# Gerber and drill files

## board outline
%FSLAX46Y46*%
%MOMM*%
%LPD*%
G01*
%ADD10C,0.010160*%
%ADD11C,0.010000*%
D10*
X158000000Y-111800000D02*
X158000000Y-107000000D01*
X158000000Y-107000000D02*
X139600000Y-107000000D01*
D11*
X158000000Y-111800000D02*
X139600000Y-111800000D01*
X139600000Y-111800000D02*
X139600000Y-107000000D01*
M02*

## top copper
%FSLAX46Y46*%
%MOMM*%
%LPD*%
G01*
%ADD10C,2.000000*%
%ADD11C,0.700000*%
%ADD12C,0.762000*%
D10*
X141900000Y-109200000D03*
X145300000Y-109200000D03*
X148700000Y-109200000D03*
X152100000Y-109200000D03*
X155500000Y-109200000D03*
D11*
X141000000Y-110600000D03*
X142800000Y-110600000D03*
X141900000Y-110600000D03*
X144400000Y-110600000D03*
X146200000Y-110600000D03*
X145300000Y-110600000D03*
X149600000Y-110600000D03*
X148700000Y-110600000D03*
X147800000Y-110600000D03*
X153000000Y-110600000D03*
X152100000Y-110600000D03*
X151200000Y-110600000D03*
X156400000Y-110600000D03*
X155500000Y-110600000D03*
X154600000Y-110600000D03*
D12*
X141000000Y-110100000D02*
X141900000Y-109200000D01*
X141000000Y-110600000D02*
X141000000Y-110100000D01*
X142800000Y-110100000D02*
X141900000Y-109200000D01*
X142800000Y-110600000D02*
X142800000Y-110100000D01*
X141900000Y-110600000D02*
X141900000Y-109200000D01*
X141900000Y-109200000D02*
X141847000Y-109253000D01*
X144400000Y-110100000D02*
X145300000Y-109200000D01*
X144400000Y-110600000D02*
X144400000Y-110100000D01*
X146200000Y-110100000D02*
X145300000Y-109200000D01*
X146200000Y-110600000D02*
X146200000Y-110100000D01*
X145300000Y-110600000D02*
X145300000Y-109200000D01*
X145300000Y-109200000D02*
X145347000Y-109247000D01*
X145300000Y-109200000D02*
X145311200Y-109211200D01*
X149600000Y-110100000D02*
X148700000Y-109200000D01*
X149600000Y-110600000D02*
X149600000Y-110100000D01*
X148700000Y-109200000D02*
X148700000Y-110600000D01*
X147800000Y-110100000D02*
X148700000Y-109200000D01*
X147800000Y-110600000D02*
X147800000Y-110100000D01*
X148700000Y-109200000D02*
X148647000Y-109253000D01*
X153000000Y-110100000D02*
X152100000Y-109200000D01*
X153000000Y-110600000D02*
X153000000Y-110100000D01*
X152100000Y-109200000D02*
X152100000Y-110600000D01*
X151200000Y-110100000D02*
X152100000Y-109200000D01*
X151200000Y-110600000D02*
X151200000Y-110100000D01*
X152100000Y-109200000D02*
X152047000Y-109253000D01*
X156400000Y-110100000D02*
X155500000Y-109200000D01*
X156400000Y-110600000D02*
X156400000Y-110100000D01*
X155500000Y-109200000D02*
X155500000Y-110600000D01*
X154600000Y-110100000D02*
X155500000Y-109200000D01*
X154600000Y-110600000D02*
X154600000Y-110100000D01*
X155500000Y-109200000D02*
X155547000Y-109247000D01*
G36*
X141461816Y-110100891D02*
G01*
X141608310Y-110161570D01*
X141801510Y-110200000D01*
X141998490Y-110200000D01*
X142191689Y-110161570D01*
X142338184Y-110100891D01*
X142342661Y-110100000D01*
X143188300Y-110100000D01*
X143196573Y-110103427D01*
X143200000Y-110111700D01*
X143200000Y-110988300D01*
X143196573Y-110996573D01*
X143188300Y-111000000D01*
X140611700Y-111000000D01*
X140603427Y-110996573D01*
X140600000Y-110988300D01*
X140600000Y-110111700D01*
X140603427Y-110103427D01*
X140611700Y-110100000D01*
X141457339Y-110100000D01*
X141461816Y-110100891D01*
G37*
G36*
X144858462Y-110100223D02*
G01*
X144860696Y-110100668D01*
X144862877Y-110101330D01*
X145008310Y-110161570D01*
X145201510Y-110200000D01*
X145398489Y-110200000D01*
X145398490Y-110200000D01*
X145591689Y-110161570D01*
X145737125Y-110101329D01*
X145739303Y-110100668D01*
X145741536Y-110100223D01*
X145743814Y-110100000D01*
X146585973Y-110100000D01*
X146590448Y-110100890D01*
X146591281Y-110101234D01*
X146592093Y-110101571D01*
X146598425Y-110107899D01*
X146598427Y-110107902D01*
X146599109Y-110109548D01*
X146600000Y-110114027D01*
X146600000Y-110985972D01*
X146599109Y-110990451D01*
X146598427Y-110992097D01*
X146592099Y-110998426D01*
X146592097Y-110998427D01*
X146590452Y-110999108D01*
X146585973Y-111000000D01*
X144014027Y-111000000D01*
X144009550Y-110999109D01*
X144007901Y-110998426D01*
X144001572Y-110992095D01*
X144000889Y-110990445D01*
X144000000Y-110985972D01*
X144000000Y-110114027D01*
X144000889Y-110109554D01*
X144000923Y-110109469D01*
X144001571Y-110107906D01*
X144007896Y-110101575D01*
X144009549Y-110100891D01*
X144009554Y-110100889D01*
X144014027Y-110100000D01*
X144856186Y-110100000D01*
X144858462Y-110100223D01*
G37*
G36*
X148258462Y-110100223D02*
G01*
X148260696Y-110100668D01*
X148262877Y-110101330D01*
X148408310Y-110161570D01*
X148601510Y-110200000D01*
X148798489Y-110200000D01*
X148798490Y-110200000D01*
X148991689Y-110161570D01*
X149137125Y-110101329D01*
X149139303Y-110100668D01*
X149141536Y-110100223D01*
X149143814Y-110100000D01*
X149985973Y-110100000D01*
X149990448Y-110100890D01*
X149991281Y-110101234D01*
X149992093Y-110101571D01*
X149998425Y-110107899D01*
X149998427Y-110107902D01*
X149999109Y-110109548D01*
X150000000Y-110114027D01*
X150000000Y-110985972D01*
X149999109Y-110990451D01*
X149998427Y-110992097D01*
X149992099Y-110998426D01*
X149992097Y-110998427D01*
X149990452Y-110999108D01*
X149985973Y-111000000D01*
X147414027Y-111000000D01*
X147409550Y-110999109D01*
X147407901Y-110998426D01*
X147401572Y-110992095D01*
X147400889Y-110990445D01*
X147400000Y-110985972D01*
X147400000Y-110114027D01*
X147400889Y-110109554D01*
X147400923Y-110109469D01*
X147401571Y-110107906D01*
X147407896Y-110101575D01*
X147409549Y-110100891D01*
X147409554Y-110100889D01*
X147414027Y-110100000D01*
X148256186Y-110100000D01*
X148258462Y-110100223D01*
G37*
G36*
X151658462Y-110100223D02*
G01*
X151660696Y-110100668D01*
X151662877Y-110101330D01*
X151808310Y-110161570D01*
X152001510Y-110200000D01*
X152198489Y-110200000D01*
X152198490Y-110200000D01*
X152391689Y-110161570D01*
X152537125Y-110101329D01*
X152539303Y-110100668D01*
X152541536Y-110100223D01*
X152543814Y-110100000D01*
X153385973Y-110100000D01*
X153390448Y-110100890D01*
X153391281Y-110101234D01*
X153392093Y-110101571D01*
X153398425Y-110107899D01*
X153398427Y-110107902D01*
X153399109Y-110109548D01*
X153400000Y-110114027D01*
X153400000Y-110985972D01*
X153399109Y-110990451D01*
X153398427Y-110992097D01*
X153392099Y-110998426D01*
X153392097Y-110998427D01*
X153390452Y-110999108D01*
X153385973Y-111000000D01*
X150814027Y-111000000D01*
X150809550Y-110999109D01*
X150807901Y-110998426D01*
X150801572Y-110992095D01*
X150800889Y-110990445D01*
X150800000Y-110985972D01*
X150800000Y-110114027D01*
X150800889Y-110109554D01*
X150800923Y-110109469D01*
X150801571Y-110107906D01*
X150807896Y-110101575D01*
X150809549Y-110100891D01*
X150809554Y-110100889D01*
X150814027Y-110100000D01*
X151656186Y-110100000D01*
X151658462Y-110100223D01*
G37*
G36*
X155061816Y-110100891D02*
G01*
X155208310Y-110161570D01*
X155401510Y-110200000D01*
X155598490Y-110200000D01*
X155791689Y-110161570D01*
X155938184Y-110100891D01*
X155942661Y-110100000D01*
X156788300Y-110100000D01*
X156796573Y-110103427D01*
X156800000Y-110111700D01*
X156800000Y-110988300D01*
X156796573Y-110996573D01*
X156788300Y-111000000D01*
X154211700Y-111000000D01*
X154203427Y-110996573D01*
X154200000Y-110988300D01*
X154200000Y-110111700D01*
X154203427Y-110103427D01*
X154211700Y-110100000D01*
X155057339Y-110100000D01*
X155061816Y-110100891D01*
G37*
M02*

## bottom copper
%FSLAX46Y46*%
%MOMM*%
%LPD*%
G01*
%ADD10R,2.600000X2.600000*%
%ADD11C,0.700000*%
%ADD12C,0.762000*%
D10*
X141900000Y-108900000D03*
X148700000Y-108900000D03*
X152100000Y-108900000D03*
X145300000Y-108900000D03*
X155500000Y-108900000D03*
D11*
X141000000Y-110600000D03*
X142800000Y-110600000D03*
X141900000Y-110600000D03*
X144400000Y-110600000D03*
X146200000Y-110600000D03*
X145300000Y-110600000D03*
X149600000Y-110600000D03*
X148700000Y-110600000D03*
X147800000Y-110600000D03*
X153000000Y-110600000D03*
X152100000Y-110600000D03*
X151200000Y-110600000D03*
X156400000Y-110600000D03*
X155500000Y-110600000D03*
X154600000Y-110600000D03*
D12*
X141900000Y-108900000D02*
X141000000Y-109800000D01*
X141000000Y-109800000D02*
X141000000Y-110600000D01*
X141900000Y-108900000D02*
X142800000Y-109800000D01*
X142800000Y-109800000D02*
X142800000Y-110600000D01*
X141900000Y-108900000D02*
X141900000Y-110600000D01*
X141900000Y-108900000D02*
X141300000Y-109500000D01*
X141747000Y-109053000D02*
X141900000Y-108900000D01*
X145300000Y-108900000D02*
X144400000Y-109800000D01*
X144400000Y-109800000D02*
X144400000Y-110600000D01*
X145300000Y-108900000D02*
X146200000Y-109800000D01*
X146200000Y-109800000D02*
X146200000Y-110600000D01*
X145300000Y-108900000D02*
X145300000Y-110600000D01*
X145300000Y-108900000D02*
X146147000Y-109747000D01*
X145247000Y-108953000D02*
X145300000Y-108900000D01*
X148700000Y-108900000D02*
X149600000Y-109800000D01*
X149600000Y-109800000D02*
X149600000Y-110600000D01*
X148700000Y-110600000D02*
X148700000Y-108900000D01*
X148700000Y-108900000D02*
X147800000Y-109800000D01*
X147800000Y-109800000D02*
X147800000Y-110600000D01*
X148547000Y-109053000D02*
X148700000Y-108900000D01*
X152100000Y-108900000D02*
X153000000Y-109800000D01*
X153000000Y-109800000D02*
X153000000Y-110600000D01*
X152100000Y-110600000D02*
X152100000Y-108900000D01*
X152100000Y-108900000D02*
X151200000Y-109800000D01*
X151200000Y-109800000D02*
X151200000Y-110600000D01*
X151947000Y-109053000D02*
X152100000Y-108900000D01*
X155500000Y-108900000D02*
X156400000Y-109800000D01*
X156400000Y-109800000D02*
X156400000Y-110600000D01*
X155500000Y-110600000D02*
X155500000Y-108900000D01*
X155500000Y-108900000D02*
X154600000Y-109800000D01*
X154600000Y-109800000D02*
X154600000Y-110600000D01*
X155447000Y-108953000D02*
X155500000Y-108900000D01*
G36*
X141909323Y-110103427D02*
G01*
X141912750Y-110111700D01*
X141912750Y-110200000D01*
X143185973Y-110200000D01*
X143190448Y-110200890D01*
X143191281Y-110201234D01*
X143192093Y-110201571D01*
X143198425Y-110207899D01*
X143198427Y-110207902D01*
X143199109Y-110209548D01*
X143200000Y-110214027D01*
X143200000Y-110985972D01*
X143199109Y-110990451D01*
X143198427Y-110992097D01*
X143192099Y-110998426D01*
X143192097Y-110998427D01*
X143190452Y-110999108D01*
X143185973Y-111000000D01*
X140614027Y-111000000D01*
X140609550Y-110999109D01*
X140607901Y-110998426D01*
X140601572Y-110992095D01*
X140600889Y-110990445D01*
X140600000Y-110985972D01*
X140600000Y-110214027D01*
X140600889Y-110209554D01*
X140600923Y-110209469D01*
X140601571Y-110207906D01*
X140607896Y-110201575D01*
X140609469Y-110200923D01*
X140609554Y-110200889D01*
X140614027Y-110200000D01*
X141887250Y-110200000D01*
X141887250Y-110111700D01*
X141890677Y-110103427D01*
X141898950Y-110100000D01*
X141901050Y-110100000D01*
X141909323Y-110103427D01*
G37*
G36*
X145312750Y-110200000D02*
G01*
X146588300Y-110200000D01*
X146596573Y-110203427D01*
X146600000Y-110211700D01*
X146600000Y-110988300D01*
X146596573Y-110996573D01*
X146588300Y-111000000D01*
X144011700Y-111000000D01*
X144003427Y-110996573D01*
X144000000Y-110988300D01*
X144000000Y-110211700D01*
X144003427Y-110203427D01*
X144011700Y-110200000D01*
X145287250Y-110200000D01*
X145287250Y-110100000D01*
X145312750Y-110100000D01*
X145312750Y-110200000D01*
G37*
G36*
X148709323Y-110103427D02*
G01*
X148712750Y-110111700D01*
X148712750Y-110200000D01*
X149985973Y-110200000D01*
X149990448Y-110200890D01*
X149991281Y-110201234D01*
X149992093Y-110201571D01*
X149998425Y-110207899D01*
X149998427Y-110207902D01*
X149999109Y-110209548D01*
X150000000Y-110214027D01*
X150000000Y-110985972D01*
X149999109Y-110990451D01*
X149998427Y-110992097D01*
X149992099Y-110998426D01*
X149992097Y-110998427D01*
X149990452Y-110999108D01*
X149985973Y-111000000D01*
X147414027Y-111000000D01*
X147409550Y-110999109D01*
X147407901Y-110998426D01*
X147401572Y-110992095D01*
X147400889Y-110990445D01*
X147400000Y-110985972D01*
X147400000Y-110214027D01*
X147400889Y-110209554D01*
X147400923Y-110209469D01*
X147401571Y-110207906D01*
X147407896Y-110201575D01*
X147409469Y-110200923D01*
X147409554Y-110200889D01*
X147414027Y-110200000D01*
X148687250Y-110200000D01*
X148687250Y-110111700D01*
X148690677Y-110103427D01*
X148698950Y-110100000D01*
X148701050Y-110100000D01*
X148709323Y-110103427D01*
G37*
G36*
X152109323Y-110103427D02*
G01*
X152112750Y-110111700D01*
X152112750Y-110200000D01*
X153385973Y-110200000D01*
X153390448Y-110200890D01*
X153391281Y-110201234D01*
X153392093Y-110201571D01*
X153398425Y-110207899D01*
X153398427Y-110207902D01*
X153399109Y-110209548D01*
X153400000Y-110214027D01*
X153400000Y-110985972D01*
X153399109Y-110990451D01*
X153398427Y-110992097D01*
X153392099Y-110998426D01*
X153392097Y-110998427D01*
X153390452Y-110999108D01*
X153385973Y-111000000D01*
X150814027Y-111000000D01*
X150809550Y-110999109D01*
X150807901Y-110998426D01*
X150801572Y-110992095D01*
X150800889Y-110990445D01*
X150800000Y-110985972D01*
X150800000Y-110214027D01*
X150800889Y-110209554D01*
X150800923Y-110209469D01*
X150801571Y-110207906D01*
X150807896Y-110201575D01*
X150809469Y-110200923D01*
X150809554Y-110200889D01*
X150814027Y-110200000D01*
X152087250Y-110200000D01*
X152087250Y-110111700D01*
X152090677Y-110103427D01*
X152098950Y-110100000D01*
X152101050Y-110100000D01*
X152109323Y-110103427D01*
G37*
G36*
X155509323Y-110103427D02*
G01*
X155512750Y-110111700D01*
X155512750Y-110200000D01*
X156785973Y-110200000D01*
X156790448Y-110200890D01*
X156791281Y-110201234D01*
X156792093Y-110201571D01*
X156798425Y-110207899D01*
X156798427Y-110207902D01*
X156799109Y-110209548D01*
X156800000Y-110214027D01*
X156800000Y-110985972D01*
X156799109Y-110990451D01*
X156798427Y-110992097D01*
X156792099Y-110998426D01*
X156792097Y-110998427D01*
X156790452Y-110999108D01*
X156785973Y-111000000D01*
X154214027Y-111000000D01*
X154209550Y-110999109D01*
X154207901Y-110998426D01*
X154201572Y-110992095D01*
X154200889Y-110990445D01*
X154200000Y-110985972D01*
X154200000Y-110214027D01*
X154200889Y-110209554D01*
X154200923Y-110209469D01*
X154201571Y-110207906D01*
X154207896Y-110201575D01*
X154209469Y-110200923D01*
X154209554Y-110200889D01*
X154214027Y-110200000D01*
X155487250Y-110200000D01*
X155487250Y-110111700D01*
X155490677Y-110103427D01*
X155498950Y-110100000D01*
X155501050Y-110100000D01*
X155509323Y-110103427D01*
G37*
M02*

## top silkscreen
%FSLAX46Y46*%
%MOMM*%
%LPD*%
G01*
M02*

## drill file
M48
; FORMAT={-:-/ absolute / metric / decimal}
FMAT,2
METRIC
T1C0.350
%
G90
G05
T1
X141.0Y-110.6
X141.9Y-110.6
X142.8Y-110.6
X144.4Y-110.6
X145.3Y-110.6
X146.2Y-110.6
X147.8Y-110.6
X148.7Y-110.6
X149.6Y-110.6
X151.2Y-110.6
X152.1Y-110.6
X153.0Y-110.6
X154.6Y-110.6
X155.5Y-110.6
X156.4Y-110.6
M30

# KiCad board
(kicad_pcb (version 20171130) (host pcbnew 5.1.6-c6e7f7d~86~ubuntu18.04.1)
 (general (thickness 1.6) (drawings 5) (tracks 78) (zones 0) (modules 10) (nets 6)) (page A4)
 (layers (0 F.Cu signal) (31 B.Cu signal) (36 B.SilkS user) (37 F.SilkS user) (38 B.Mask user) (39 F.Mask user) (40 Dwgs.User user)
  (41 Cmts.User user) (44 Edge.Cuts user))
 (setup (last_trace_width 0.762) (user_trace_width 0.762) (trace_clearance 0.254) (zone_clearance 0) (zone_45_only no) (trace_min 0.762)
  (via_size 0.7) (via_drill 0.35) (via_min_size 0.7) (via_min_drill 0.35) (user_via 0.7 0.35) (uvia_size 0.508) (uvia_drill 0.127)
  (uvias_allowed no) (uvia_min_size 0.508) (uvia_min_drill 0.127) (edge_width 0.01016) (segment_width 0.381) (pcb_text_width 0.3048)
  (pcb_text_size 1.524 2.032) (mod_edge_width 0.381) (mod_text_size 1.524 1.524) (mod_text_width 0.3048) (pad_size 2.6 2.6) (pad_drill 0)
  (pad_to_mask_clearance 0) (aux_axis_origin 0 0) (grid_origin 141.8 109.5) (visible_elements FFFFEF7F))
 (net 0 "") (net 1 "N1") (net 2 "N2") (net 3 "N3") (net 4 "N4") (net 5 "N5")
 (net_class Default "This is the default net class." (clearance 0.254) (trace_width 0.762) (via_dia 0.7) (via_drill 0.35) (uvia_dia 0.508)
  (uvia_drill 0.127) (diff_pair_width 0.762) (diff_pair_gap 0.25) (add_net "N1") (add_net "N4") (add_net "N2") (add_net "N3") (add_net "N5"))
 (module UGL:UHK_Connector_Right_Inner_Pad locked (layer B.Cu) (at 146.31 108.9)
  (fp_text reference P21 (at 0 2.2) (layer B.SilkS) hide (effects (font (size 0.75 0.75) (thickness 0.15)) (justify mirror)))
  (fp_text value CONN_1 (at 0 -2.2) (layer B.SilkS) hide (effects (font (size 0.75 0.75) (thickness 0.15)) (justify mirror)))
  (pad 1 smd rect (at -4.41 0) (size 2.6 2.6) (layers B.Cu B.Mask) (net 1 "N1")))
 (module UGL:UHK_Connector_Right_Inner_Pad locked (layer B.Cu) (at 151.15 108.9)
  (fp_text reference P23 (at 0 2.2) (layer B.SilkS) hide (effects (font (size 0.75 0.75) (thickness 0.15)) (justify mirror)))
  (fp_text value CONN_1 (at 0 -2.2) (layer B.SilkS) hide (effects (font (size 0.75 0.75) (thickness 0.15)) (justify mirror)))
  (pad 1 smd rect (at -2.45 0) (size 2.6 2.6) (layers B.Cu B.Mask) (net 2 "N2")))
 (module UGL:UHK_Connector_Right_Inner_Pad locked (layer B.Cu) (at 153.57 108.9)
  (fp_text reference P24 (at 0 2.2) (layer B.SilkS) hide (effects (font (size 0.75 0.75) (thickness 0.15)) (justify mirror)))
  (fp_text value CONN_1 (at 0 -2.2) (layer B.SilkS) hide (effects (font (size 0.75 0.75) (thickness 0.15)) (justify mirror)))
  (pad 1 smd rect (at -1.47 0) (size 2.6 2.6) (layers B.Cu B.Mask) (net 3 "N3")))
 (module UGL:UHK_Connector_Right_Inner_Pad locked (layer B.Cu) (at 148.73 108.9)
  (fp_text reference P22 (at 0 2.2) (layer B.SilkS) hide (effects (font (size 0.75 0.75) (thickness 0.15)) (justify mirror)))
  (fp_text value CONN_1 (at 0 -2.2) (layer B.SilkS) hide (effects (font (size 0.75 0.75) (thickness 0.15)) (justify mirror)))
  (pad 1 smd rect (at -3.43 0) (size 2.6 2.6) (layers B.Cu B.Mask) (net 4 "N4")))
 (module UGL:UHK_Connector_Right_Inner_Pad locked (layer B.Cu) (at 155.99 108.9)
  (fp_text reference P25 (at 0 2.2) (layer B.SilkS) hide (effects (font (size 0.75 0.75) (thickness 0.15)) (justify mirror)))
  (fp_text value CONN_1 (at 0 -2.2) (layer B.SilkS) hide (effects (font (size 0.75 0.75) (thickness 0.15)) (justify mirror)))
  (pad 1 smd rect (at -0.49 0) (size 2.6 2.6) (layers B.Cu B.Mask) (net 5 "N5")))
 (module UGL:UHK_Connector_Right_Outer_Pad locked (layer F.Cu) (at 141.9 109.2)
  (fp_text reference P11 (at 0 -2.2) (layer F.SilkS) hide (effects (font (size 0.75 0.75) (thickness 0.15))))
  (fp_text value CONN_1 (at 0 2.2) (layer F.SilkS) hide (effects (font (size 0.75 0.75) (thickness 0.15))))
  (pad 1 smd circle (at 0 0) (size 2 2) (layers F.Cu F.Mask) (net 1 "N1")))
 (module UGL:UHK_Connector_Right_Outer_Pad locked (layer F.Cu) (at 145.3 109.2)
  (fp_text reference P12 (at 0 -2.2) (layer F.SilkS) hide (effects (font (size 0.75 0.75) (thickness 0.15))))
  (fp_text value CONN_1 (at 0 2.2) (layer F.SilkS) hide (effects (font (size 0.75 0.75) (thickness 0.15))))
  (pad 1 smd circle (at 0 0) (size 2 2) (layers F.Cu F.Mask) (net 4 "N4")))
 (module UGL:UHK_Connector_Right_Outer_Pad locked (layer F.Cu) (at 148.7 109.2)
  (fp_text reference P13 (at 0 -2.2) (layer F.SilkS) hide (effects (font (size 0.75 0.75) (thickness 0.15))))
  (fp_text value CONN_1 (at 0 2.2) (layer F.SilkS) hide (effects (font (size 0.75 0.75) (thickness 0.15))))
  (pad 1 smd circle (at 0 0) (size 2 2) (layers F.Cu F.Mask) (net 2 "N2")))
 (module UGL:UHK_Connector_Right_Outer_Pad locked (layer F.Cu) (at 152.1 109.2)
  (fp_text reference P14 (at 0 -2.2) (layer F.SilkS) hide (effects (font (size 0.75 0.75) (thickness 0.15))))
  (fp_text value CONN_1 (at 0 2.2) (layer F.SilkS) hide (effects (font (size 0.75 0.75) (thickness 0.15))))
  (pad 1 smd circle (at 0 0) (size 2 2) (layers F.Cu F.Mask) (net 3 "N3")))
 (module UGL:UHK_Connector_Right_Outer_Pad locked (layer F.Cu) (at 155.5 109.2)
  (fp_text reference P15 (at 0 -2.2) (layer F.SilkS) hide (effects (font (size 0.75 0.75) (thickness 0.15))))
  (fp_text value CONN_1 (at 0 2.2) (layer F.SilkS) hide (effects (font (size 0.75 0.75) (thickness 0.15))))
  (pad 1 smd circle (at 0 0) (size 2 2) (layers F.Cu F.Mask) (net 5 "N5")))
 (gr_line (start 158 111.8) (end 158 107) (layer Edge.Cuts) (width 0.01016))
 (gr_line (start 158 107) (end 139.6 107) (layer Edge.Cuts) (width 0.01016))
 (gr_line (start 158 111.8) (end 139.6 111.8) (angle 90) (layer Edge.Cuts) (width 0.01))
 (gr_line (start 139.6 111.8) (end 139.6 107) (angle 90) (layer Edge.Cuts) (width 0.01))
 (segment (start 141.9 108.9) (end 141 109.8) (width 0.762) (layer B.Cu) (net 1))
 (segment (start 141 109.8) (end 141 110.6) (width 0.762) (layer B.Cu) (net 1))
 (segment (start 141 110.1) (end 141.9 109.2) (width 0.762) (layer F.Cu) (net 1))
 (segment (start 141 110.6) (end 141 110.1) (width 0.762) (layer F.Cu) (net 1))
 (via (at 141 110.6) (size 0.7) (drill 0.35) (layers F.Cu B.Cu) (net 1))
 (segment (start 141.9 108.9) (end 142.8 109.8) (width 0.762) (layer B.Cu) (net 1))
 (segment (start 142.8 109.8) (end 142.8 110.6) (width 0.762) (layer B.Cu) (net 1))
 (segment (start 142.8 110.1) (end 141.9 109.2) (width 0.762) (layer F.Cu) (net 1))
 (segment (start 142.8 110.6) (end 142.8 110.1) (width 0.762) (layer F.Cu) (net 1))
 (via (at 142.8 110.6) (size 0.7) (drill 0.35) (layers F.Cu B.Cu) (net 1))
 (segment (start 141.9 108.9) (end 141.9 110.6) (width 0.762) (layer B.Cu) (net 1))
 (segment (start 141.9 110.6) (end 141.9 109.2) (width 0.762) (layer F.Cu) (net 1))
 (via (at 141.9 110.6) (size 0.7) (drill 0.35) (layers F.Cu B.Cu) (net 1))
 (segment (start 141.9 108.9) (end 141.3 109.5) (width 0.762) (layer B.Cu) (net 1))
 (segment (start 141.9 109.2) (end 141.847 109.253) (width 0.762) (layer F.Cu) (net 1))
 (segment (start 141.747 109.053) (end 141.9 108.9) (width 0.762) (layer B.Cu) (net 1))
 (segment (start 145.3 108.9) (end 144.4 109.8) (width 0.762) (layer B.Cu) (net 4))
 (segment (start 144.4 109.8) (end 144.4 110.6) (width 0.762) (layer B.Cu) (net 4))
 (segment (start 144.4 110.1) (end 145.3 109.2) (width 0.762) (layer F.Cu) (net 4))
 (segment (start 144.4 110.6) (end 144.4 110.1) (width 0.762) (layer F.Cu) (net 4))
 (via (at 144.4 110.6) (size 0.7) (drill 0.35) (layers F.Cu B.Cu) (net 4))
 (segment (start 145.3 108.9) (end 146.2 109.8) (width 0.762) (layer B.Cu) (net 4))
 (segment (start 146.2 109.8) (end 146.2 110.6) (width 0.762) (layer B.Cu) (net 4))
 (segment (start 146.2 110.1) (end 145.3 109.2) (width 0.762) (layer F.Cu) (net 4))
 (segment (start 146.2 110.6) (end 146.2 110.1) (width 0.762) (layer F.Cu) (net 4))
 (via (at 146.2 110.6) (size 0.7) (drill 0.35) (layers F.Cu B.Cu) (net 4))
 (segment (start 145.3 108.9) (end 145.3 110.6) (width 0.762) (layer B.Cu) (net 4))
 (segment (start 145.3 110.6) (end 145.3 109.2) (width 0.762) (layer F.Cu) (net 4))
 (via (at 145.3 110.6) (size 0.7) (drill 0.35) (layers F.Cu B.Cu) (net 4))
 (segment (start 145.3 108.9) (end 146.147 109.747) (width 0.762) (layer B.Cu) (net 4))
 (segment (start 145.3 109.2) (end 145.347 109.247) (width 0.762) (layer F.Cu) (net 4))
 (segment (start 145.247 108.953) (end 145.3 108.9) (width 0.762) (layer B.Cu) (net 4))
 (segment (start 145.3 109.2) (end 145.3112 109.2112) (width 0.762) (layer F.Cu) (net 4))
 (segment (start 148.7 108.9) (end 149.6 109.8) (width 0.762) (layer B.Cu) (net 2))
 (segment (start 149.6 109.8) (end 149.6 110.6) (width 0.762) (layer B.Cu) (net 2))
 (segment (start 149.6 110.1) (end 148.7 109.2) (width 0.762) (layer F.Cu) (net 2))
 (segment (start 149.6 110.6) (end 149.6 110.1) (width 0.762) (layer F.Cu) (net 2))
 (via (at 149.6 110.6) (size 0.7) (drill 0.35) (layers F.Cu B.Cu) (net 2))
 (segment (start 148.7 109.2) (end 148.7 110.6) (width 0.762) (layer F.Cu) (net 2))
 (segment (start 148.7 110.6) (end 148.7 108.9) (width 0.762) (layer B.Cu) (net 2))
 (via (at 148.7 110.6) (size 0.7) (drill 0.35) (layers F.Cu B.Cu) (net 2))
 (segment (start 148.7 108.9) (end 147.8 109.8) (width 0.762) (layer B.Cu) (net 2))
 (segment (start 147.8 109.8) (end 147.8 110.6) (width 0.762) (layer B.Cu) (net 2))
 (segment (start 147.8 110.1) (end 148.7 109.2) (width 0.762) (layer F.Cu) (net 2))
 (segment (start 147.8 110.6) (end 147.8 110.1) (width 0.762) (layer F.Cu) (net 2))
 (via (at 147.8 110.6) (size 0.7) (drill 0.35) (layers F.Cu B.Cu) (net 2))
 (segment (start 148.7 109.2) (end 148.647 109.253) (width 0.762) (layer F.Cu) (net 2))
 (segment (start 148.547 109.053) (end 148.7 108.9) (width 0.762) (layer B.Cu) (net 2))
 (segment (start 152.1 108.9) (end 153 109.8) (width 0.762) (layer B.Cu) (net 3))
 (segment (start 153 109.8) (end 153 110.6) (width 0.762) (layer B.Cu) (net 3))
 (segment (start 153 110.1) (end 152.1 109.2) (width 0.762) (layer F.Cu) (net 3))
 (segment (start 153 110.6) (end 153 110.1) (width 0.762) (layer F.Cu) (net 3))
 (via (at 153 110.6) (size 0.7) (drill 0.35) (layers F.Cu B.Cu) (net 3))
 (segment (start 152.1 109.2) (end 152.1 110.6) (width 0.762) (layer F.Cu) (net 3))
 (segment (start 152.1 110.6) (end 152.1 108.9) (width 0.762) (layer B.Cu) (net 3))
 (via (at 152.1 110.6) (size 0.7) (drill 0.35) (layers F.Cu B.Cu) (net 3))
 (segment (start 152.1 108.9) (end 151.2 109.8) (width 0.762) (layer B.Cu) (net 3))
 (segment (start 151.2 109.8) (end 151.2 110.6) (width 0.762) (layer B.Cu) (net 3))
 (segment (start 151.2 110.1) (end 152.1 109.2) (width 0.762) (layer F.Cu) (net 3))
 (segment (start 151.2 110.6) (end 151.2 110.1) (width 0.762) (layer F.Cu) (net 3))
 (via (at 151.2 110.6) (size 0.7) (drill 0.35) (layers F.Cu B.Cu) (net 3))
 (segment (start 152.1 109.2) (end 152.047 109.253) (width 0.762) (layer F.Cu) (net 3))
 (segment (start 151.947 109.053) (end 152.1 108.9) (width 0.762) (layer B.Cu) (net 3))
 (segment (start 155.5 108.9) (end 156.4 109.8) (width 0.762) (layer B.Cu) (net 5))
 (segment (start 156.4 109.8) (end 156.4 110.6) (width 0.762) (layer B.Cu) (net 5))
 (segment (start 156.4 110.1) (end 155.5 109.2) (width 0.762) (layer F.Cu) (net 5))
 (segment (start 156.4 110.6) (end 156.4 110.1) (width 0.762) (layer F.Cu) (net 5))
 (via (at 156.4 110.6) (size 0.7) (drill 0.35) (layers F.Cu B.Cu) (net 5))
 (segment (start 155.5 109.2) (end 155.5 110.6) (width 0.762) (layer F.Cu) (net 5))
 (segment (start 155.5 110.6) (end 155.5 108.9) (width 0.762) (layer B.Cu) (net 5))
 (via (at 155.5 110.6) (size 0.7) (drill 0.35) (layers F.Cu B.Cu) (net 5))
 (segment (start 155.5 108.9) (end 154.6 109.8) (width 0.762) (layer B.Cu) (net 5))
 (segment (start 154.6 109.8) (end 154.6 110.6) (width 0.762) (layer B.Cu) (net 5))
 (segment (start 154.6 110.1) (end 155.5 109.2) (width 0.762) (layer F.Cu) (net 5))
 (segment (start 154.6 110.6) (end 154.6 110.1) (width 0.762) (layer F.Cu) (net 5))
 (via (at 154.6 110.6) (size 0.7) (drill 0.35) (layers F.Cu B.Cu) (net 5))
 (segment (start 155.5 109.2) (end 155.547 109.247) (width 0.762) (layer F.Cu) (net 5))
 (segment (start 155.447 108.953) (end 155.5 108.9) (width 0.762) (layer B.Cu) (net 5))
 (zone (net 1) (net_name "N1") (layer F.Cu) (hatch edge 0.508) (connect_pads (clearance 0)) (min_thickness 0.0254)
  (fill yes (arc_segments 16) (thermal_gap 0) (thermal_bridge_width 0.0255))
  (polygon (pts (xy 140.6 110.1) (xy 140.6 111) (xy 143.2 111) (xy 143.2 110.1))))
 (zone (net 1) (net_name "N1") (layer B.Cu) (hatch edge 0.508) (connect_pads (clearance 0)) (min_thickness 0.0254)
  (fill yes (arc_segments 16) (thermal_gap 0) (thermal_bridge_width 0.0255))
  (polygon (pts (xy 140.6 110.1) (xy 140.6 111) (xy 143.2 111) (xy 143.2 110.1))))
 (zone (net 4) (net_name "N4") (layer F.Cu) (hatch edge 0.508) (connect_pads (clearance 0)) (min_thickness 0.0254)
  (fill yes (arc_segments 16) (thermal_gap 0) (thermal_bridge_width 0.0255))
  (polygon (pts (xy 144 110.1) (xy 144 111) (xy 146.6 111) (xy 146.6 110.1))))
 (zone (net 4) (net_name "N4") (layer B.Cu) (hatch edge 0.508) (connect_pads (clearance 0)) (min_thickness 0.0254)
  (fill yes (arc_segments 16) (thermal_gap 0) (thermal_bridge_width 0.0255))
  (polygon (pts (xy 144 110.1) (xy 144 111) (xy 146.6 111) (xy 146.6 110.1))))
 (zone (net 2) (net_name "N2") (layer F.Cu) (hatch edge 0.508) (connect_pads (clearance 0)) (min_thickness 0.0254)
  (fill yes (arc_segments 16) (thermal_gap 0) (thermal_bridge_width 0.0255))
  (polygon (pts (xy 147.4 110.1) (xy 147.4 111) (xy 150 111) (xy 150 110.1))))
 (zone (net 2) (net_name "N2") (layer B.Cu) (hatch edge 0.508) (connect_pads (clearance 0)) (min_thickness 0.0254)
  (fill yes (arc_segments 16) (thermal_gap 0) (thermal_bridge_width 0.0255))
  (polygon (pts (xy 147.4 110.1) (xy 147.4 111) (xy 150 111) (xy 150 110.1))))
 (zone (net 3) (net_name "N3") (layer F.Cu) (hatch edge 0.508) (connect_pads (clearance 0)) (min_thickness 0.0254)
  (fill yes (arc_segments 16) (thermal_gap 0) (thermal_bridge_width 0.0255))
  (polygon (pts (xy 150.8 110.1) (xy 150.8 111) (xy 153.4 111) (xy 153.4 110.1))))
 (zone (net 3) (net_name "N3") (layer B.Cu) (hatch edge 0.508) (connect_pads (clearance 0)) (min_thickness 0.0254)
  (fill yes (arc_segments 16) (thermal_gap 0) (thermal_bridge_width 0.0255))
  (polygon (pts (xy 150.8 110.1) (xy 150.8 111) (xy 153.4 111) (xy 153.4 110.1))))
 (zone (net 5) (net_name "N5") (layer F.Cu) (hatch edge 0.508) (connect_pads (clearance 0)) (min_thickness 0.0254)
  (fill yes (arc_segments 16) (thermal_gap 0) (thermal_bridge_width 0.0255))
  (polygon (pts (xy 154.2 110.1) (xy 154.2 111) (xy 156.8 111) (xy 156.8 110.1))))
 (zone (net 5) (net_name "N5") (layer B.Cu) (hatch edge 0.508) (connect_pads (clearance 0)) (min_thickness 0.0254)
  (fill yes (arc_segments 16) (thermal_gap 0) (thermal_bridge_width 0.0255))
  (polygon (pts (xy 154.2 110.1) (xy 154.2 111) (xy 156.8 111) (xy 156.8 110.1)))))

